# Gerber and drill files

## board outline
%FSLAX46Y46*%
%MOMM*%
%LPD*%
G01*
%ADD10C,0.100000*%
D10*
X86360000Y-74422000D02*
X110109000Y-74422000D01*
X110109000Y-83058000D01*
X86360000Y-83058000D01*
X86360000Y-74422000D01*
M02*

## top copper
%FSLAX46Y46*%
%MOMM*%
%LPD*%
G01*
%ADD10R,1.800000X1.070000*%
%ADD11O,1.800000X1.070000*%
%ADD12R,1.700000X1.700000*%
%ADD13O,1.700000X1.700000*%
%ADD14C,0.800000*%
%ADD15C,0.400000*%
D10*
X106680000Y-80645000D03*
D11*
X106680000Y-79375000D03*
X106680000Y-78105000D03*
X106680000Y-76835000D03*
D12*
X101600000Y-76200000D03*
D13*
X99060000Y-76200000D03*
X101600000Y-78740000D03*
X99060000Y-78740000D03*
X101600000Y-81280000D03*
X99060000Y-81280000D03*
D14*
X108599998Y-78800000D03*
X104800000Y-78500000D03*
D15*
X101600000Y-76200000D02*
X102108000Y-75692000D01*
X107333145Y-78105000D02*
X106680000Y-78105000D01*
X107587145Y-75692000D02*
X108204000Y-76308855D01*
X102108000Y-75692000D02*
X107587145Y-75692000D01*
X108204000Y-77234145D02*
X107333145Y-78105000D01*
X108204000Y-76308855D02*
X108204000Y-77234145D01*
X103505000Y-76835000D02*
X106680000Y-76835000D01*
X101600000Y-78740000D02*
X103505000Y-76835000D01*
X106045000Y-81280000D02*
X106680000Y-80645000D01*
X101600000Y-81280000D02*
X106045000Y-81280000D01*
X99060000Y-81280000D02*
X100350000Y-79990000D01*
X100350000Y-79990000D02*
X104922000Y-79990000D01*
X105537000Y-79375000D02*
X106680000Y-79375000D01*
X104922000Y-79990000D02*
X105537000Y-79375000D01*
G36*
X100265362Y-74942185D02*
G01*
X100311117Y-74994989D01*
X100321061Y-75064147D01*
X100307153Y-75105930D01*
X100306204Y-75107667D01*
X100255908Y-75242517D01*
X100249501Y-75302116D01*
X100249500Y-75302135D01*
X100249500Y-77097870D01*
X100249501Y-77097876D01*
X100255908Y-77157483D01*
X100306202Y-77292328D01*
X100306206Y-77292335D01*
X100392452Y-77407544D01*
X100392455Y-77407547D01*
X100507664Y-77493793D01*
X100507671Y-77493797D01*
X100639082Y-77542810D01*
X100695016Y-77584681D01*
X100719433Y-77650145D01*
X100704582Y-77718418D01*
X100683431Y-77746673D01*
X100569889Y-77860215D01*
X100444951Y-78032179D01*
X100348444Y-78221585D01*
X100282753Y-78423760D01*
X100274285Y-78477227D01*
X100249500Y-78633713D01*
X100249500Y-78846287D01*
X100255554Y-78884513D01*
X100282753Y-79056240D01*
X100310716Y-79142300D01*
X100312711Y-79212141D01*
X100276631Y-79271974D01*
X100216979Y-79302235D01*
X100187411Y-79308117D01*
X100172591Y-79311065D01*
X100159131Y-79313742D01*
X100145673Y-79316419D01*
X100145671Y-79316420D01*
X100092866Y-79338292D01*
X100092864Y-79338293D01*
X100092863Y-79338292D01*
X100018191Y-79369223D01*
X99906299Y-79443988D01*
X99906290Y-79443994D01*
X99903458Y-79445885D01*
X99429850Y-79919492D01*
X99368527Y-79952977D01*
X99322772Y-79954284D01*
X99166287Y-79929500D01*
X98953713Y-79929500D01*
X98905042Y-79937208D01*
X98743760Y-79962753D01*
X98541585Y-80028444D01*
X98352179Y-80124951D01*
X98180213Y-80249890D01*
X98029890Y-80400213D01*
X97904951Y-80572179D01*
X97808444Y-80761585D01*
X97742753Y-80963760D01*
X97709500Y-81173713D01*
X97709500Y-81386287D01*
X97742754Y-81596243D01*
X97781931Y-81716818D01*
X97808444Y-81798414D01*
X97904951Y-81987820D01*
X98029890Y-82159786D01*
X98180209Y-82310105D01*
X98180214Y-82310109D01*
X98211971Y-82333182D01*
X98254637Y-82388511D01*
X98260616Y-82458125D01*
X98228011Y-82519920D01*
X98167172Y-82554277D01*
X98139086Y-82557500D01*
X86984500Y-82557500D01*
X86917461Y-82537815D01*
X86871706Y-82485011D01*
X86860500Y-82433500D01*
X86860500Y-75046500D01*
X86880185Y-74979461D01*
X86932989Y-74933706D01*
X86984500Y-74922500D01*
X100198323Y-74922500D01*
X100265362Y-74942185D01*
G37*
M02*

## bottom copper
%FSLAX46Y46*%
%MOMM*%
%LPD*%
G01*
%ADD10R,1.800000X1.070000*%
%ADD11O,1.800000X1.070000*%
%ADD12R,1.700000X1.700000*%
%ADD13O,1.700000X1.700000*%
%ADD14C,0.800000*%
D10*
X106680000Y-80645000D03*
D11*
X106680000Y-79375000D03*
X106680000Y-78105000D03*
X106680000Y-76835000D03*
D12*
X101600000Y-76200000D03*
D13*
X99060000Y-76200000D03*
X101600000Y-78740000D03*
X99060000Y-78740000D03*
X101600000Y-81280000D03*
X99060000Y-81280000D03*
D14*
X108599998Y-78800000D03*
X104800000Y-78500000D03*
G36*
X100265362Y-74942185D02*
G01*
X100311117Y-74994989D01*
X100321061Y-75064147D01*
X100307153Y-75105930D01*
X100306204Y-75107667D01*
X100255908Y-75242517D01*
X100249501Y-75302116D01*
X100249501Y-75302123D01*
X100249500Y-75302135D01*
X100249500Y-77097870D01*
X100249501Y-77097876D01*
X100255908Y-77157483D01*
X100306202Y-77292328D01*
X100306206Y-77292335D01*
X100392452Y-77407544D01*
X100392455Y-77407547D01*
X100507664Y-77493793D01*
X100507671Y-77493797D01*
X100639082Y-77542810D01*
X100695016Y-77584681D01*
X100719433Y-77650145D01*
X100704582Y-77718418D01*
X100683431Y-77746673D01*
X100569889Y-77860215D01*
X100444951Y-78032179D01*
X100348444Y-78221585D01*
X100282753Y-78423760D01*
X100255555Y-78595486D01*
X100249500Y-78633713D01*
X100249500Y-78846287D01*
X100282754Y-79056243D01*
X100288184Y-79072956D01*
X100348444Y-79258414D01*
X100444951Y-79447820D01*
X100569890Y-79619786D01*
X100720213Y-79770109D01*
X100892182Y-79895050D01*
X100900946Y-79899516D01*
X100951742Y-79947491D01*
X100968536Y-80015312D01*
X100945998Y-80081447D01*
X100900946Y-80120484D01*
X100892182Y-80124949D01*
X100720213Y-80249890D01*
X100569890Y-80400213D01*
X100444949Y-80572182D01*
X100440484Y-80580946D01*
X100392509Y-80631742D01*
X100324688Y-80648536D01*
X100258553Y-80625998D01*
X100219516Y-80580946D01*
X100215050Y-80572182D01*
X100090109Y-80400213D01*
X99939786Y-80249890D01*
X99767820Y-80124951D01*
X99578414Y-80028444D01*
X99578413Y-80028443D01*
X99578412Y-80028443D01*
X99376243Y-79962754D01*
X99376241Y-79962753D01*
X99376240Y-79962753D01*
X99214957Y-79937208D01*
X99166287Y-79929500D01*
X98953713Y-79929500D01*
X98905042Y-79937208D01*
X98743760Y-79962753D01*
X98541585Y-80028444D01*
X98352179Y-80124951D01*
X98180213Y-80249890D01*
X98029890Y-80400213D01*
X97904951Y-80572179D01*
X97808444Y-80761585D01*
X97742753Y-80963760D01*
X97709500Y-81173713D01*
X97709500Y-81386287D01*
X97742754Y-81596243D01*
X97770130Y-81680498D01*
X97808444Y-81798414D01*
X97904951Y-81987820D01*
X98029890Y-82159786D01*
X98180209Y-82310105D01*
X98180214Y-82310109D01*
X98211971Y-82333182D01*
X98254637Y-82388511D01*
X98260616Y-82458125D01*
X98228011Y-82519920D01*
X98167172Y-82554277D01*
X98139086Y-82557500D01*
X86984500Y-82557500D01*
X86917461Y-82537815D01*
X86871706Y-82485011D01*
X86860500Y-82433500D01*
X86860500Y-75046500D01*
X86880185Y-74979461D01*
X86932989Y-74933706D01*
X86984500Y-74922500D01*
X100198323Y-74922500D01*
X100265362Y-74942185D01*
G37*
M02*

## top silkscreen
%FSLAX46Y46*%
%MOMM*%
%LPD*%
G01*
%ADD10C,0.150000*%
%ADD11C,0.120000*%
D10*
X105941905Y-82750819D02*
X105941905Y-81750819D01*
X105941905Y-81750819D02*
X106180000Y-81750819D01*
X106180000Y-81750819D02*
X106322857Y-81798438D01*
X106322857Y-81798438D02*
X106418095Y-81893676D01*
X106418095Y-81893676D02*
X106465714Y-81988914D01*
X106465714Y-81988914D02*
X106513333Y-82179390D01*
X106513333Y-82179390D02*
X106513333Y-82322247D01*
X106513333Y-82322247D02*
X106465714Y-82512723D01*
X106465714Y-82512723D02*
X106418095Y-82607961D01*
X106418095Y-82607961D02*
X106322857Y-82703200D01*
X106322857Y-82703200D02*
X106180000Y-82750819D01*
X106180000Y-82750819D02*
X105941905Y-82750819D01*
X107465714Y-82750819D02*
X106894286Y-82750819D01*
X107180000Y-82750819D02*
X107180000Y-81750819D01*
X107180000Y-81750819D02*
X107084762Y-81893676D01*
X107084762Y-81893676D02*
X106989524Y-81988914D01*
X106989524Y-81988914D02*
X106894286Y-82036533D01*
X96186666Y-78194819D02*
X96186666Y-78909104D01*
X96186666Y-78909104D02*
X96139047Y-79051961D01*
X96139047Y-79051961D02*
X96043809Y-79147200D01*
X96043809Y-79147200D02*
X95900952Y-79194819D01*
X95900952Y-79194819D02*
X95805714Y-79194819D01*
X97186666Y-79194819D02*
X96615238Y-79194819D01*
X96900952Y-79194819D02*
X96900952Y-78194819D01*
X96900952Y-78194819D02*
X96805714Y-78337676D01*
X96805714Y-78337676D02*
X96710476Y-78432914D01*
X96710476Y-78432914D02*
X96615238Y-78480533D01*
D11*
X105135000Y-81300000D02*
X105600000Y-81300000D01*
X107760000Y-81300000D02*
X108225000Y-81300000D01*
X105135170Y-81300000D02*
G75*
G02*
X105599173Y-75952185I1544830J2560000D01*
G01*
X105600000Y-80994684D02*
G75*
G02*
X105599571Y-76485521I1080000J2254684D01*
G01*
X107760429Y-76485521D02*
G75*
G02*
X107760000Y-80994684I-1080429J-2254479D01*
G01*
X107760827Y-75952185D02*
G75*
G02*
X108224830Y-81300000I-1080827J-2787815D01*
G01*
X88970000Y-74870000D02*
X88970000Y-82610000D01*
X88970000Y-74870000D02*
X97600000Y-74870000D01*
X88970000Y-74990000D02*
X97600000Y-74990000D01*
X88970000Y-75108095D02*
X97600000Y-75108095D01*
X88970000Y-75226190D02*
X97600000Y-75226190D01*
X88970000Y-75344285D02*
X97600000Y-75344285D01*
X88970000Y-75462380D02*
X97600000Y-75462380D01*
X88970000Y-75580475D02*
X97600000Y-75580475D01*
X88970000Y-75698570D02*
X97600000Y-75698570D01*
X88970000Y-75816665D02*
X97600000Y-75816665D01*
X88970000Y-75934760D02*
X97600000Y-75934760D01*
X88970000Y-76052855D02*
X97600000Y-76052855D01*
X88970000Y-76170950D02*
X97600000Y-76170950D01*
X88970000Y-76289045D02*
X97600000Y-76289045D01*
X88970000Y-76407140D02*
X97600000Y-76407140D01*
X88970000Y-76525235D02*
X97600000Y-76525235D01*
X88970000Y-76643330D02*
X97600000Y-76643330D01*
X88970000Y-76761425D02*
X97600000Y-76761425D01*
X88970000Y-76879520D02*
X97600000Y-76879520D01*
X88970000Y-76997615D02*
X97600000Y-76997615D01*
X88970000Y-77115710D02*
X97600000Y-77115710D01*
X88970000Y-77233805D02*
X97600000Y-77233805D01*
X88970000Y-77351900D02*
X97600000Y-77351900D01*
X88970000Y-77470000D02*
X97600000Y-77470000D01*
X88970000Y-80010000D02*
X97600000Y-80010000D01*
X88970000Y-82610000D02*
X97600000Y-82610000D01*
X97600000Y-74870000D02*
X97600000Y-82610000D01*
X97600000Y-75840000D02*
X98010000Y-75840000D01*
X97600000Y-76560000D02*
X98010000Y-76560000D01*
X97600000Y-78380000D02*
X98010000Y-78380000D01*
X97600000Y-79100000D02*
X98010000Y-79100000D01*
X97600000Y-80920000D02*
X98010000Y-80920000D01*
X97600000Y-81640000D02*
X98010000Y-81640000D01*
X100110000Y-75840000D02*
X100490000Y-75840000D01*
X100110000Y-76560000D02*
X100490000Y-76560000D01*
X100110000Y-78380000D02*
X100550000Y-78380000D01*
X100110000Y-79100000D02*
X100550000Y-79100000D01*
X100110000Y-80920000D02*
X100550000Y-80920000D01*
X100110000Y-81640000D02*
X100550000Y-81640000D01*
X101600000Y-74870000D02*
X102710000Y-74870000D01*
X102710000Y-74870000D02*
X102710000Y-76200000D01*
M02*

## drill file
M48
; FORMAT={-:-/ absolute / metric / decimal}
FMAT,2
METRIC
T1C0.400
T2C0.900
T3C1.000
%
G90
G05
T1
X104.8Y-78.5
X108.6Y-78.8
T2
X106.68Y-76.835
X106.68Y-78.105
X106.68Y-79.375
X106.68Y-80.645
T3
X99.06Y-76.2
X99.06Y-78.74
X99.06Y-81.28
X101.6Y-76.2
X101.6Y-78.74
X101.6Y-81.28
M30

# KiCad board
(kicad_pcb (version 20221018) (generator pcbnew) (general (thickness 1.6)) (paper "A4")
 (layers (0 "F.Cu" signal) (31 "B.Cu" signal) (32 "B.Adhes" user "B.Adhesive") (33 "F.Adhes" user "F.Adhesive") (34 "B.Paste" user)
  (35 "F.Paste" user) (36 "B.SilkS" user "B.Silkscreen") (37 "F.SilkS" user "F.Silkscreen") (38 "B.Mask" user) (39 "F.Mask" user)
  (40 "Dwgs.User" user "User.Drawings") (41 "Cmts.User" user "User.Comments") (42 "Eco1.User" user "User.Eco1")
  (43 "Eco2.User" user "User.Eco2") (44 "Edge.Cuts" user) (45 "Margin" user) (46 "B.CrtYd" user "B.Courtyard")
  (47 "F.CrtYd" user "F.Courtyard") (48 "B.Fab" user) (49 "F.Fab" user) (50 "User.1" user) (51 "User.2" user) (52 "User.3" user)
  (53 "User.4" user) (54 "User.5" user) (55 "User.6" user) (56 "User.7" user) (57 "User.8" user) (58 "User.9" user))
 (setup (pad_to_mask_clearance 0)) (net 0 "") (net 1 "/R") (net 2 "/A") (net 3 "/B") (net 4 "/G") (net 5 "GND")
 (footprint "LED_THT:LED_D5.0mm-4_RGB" (layer "F.Cu") (at 106.68 80.645 90)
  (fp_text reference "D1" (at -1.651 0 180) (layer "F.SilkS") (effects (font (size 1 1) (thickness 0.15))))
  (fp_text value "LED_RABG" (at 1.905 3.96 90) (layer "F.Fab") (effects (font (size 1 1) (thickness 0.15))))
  (fp_line (start -0.655 -1.545) (end -0.655 -1.08) (stroke (width 0.12) (type solid)) (layer "F.SilkS"))
  (fp_line (start -0.655 1.08) (end -0.655 1.545) (stroke (width 0.12) (type solid)) (layer "F.SilkS"))
  (fp_arc (start -0.655 -1.54483) (mid 2.163456 -2.978809) (end 4.692815 -1.080827) (stroke (width 0.12) (type solid)) (layer "F.SilkS"))
  (fp_arc (start -0.349684 -1.08) (mid 1.904762 -2.5) (end 4.159479 -1.080429) (stroke (width 0.12) (type solid)) (layer "F.SilkS"))
  (fp_arc (start 4.159479 1.080429) (mid 1.904762 2.5) (end -0.349684 1.08) (stroke (width 0.12) (type solid)) (layer "F.SilkS"))
  (fp_arc (start 4.692815 1.080827) (mid 2.163456 2.978808) (end -0.655 1.54483) (stroke (width 0.12) (type solid)) (layer "F.SilkS"))
  (pad "1" thru_hole rect (at 0 0 90) (size 1.07 1.8) (drill 0.9) (layers "*.Cu" "*.Mask") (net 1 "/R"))
  (pad "2" thru_hole oval (at 1.27 0 90) (size 1.07 1.8) (drill 0.9) (layers "*.Cu" "*.Mask") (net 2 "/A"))
  (pad "3" thru_hole oval (at 2.54 0 90) (size 1.07 1.8) (drill 0.9) (layers "*.Cu" "*.Mask") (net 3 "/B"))
  (pad "4" thru_hole oval (at 3.81 0 90) (size 1.07 1.8) (drill 0.9) (layers "*.Cu" "*.Mask") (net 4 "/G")))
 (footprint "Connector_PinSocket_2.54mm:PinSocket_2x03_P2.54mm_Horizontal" (layer "F.Cu") (at 101.6 76.2)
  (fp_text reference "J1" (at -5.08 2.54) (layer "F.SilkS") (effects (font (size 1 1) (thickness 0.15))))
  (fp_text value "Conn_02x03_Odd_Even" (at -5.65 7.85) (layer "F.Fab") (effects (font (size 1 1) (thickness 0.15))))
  (fp_line (start -12.63 -1.33) (end -12.63 6.41) (stroke (width 0.12) (type solid)) (layer "F.SilkS"))
  (fp_line (start -12.63 -1.33) (end -4 -1.33) (stroke (width 0.12) (type solid)) (layer "F.SilkS"))
  (fp_line (start -12.63 -1.21) (end -4 -1.21) (stroke (width 0.12) (type solid)) (layer "F.SilkS"))
  (fp_line (start -12.63 -1.091905) (end -4 -1.091905) (stroke (width 0.12) (type solid)) (layer "F.SilkS"))
  (fp_line (start -12.63 -0.97381) (end -4 -0.97381) (stroke (width 0.12) (type solid)) (layer "F.SilkS"))
  (fp_line (start -12.63 -0.855715) (end -4 -0.855715) (stroke (width 0.12) (type solid)) (layer "F.SilkS"))
  (fp_line (start -12.63 -0.73762) (end -4 -0.73762) (stroke (width 0.12) (type solid)) (layer "F.SilkS"))
  (fp_line (start -12.63 -0.619525) (end -4 -0.619525) (stroke (width 0.12) (type solid)) (layer "F.SilkS"))
  (fp_line (start -12.63 -0.50143) (end -4 -0.50143) (stroke (width 0.12) (type solid)) (layer "F.SilkS"))
  (fp_line (start -12.63 -0.383335) (end -4 -0.383335) (stroke (width 0.12) (type solid)) (layer "F.SilkS"))
  (fp_line (start -12.63 -0.26524) (end -4 -0.26524) (stroke (width 0.12) (type solid)) (layer "F.SilkS"))
  (fp_line (start -12.63 -0.147145) (end -4 -0.147145) (stroke (width 0.12) (type solid)) (layer "F.SilkS"))
  (fp_line (start -12.63 -0.02905) (end -4 -0.02905) (stroke (width 0.12) (type solid)) (layer "F.SilkS"))
  (fp_line (start -12.63 0.089045) (end -4 0.089045) (stroke (width 0.12) (type solid)) (layer "F.SilkS"))
  (fp_line (start -12.63 0.20714) (end -4 0.20714) (stroke (width 0.12) (type solid)) (layer "F.SilkS"))
  (fp_line (start -12.63 0.325235) (end -4 0.325235) (stroke (width 0.12) (type solid)) (layer "F.SilkS"))
  (fp_line (start -12.63 0.44333) (end -4 0.44333) (stroke (width 0.12) (type solid)) (layer "F.SilkS"))
  (fp_line (start -12.63 0.561425) (end -4 0.561425) (stroke (width 0.12) (type solid)) (layer "F.SilkS"))
  (fp_line (start -12.63 0.67952) (end -4 0.67952) (stroke (width 0.12) (type solid)) (layer "F.SilkS"))
  (fp_line (start -12.63 0.797615) (end -4 0.797615) (stroke (width 0.12) (type solid)) (layer "F.SilkS"))
  (fp_line (start -12.63 0.91571) (end -4 0.91571) (stroke (width 0.12) (type solid)) (layer "F.SilkS"))
  (fp_line (start -12.63 1.033805) (end -4 1.033805) (stroke (width 0.12) (type solid)) (layer "F.SilkS"))
  (fp_line (start -12.63 1.1519) (end -4 1.1519) (stroke (width 0.12) (type solid)) (layer "F.SilkS"))
  (fp_line (start -12.63 1.27) (end -4 1.27) (stroke (width 0.12) (type solid)) (layer "F.SilkS"))
  (fp_line (start -12.63 3.81) (end -4 3.81) (stroke (width 0.12) (type solid)) (layer "F.SilkS"))
  (fp_line (start -12.63 6.41) (end -4 6.41) (stroke (width 0.12) (type solid)) (layer "F.SilkS"))
  (fp_line (start -4 -1.33) (end -4 6.41) (stroke (width 0.12) (type solid)) (layer "F.SilkS"))
  (fp_line (start -4 -0.36) (end -3.59 -0.36) (stroke (width 0.12) (type solid)) (layer "F.SilkS"))
  (fp_line (start -4 0.36) (end -3.59 0.36) (stroke (width 0.12) (type solid)) (layer "F.SilkS"))
  (fp_line (start -4 2.18) (end -3.59 2.18) (stroke (width 0.12) (type solid)) (layer "F.SilkS"))
  (fp_line (start -4 2.9) (end -3.59 2.9) (stroke (width 0.12) (type solid)) (layer "F.SilkS"))
  (fp_line (start -4 4.72) (end -3.59 4.72) (stroke (width 0.12) (type solid)) (layer "F.SilkS"))
  (fp_line (start -4 5.44) (end -3.59 5.44) (stroke (width 0.12) (type solid)) (layer "F.SilkS"))
  (fp_line (start -1.49 -0.36) (end -1.11 -0.36) (stroke (width 0.12) (type solid)) (layer "F.SilkS"))
  (fp_line (start -1.49 0.36) (end -1.11 0.36) (stroke (width 0.12) (type solid)) (layer "F.SilkS"))
  (fp_line (start -1.49 2.18) (end -1.05 2.18) (stroke (width 0.12) (type solid)) (layer "F.SilkS"))
  (fp_line (start -1.49 2.9) (end -1.05 2.9) (stroke (width 0.12) (type solid)) (layer "F.SilkS"))
  (fp_line (start -1.49 4.72) (end -1.05 4.72) (stroke (width 0.12) (type solid)) (layer "F.SilkS"))
  (fp_line (start -1.49 5.44) (end -1.05 5.44) (stroke (width 0.12) (type solid)) (layer "F.SilkS"))
  (fp_line (start 0 -1.33) (end 1.11 -1.33) (stroke (width 0.12) (type solid)) (layer "F.SilkS"))
  (fp_line (start 1.11 -1.33) (end 1.11 0) (stroke (width 0.12) (type solid)) (layer "F.SilkS"))
  (pad "1" thru_hole rect (at 0 0) (size 1.7 1.7) (drill 1) (layers "*.Cu" "*.Mask") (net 3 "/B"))
  (pad "2" thru_hole oval (at -2.54 0) (size 1.7 1.7) (drill 1) (layers "*.Cu" "*.Mask") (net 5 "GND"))
  (pad "3" thru_hole oval (at 0 2.54) (size 1.7 1.7) (drill 1) (layers "*.Cu" "*.Mask") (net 4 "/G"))
  (pad "4" thru_hole oval (at -2.54 2.54) (size 1.7 1.7) (drill 1) (layers "*.Cu" "*.Mask") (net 5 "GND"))
  (pad "5" thru_hole oval (at 0 5.08) (size 1.7 1.7) (drill 1) (layers "*.Cu" "*.Mask") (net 1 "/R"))
  (pad "6" thru_hole oval (at -2.54 5.08) (size 1.7 1.7) (drill 1) (layers "*.Cu" "*.Mask") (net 2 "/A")))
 (gr_rect (start 86.36 74.422) (end 110.109 83.058) (stroke (width 0.1) (type default)) (fill none) (layer "Edge.Cuts"))
 (segment (start 101.6 76.2) (end 102.108 75.692) (width 0.4) (layer "F.Cu") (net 3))
 (segment (start 107.333145 78.105) (end 106.68 78.105) (width 0.4) (layer "F.Cu") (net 3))
 (segment (start 107.587145 75.692) (end 108.204 76.308855) (width 0.4) (layer "F.Cu") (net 3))
 (segment (start 102.108 75.692) (end 107.587145 75.692) (width 0.4) (layer "F.Cu") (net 3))
 (segment (start 108.204 77.234145) (end 107.333145 78.105) (width 0.4) (layer "F.Cu") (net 3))
 (segment (start 108.204 76.308855) (end 108.204 77.234145) (width 0.4) (layer "F.Cu") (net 3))
 (via (at 108.599998 78.8) (size 0.8) (drill 0.4) (layers "F.Cu" "B.Cu") (free) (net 5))
 (via (at 104.8 78.5) (size 0.8) (drill 0.4) (layers "F.Cu" "B.Cu") (free) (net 5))
 (segment (start 103.505 76.835) (end 106.68 76.835) (width 0.4) (layer "F.Cu") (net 4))
 (segment (start 101.6 78.74) (end 103.505 76.835) (width 0.4) (layer "F.Cu") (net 4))
 (segment (start 106.045 81.28) (end 106.68 80.645) (width 0.4) (layer "F.Cu") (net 1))
 (segment (start 101.6 81.28) (end 106.045 81.28) (width 0.4) (layer "F.Cu") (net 1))
 (segment (start 99.06 81.28) (end 100.35 79.99) (width 0.4) (layer "F.Cu") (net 2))
 (segment (start 100.35 79.99) (end 104.922 79.99) (width 0.4) (layer "F.Cu") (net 2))
 (segment (start 105.537 79.375) (end 106.68 79.375) (width 0.4) (layer "F.Cu") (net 2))
 (segment (start 104.922 79.99) (end 105.537 79.375) (width 0.4) (layer "F.Cu") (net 2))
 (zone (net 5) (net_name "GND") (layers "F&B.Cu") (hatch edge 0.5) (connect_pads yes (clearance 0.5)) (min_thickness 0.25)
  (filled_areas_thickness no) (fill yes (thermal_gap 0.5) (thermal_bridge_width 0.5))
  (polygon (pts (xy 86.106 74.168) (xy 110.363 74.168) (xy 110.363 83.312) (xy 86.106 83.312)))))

